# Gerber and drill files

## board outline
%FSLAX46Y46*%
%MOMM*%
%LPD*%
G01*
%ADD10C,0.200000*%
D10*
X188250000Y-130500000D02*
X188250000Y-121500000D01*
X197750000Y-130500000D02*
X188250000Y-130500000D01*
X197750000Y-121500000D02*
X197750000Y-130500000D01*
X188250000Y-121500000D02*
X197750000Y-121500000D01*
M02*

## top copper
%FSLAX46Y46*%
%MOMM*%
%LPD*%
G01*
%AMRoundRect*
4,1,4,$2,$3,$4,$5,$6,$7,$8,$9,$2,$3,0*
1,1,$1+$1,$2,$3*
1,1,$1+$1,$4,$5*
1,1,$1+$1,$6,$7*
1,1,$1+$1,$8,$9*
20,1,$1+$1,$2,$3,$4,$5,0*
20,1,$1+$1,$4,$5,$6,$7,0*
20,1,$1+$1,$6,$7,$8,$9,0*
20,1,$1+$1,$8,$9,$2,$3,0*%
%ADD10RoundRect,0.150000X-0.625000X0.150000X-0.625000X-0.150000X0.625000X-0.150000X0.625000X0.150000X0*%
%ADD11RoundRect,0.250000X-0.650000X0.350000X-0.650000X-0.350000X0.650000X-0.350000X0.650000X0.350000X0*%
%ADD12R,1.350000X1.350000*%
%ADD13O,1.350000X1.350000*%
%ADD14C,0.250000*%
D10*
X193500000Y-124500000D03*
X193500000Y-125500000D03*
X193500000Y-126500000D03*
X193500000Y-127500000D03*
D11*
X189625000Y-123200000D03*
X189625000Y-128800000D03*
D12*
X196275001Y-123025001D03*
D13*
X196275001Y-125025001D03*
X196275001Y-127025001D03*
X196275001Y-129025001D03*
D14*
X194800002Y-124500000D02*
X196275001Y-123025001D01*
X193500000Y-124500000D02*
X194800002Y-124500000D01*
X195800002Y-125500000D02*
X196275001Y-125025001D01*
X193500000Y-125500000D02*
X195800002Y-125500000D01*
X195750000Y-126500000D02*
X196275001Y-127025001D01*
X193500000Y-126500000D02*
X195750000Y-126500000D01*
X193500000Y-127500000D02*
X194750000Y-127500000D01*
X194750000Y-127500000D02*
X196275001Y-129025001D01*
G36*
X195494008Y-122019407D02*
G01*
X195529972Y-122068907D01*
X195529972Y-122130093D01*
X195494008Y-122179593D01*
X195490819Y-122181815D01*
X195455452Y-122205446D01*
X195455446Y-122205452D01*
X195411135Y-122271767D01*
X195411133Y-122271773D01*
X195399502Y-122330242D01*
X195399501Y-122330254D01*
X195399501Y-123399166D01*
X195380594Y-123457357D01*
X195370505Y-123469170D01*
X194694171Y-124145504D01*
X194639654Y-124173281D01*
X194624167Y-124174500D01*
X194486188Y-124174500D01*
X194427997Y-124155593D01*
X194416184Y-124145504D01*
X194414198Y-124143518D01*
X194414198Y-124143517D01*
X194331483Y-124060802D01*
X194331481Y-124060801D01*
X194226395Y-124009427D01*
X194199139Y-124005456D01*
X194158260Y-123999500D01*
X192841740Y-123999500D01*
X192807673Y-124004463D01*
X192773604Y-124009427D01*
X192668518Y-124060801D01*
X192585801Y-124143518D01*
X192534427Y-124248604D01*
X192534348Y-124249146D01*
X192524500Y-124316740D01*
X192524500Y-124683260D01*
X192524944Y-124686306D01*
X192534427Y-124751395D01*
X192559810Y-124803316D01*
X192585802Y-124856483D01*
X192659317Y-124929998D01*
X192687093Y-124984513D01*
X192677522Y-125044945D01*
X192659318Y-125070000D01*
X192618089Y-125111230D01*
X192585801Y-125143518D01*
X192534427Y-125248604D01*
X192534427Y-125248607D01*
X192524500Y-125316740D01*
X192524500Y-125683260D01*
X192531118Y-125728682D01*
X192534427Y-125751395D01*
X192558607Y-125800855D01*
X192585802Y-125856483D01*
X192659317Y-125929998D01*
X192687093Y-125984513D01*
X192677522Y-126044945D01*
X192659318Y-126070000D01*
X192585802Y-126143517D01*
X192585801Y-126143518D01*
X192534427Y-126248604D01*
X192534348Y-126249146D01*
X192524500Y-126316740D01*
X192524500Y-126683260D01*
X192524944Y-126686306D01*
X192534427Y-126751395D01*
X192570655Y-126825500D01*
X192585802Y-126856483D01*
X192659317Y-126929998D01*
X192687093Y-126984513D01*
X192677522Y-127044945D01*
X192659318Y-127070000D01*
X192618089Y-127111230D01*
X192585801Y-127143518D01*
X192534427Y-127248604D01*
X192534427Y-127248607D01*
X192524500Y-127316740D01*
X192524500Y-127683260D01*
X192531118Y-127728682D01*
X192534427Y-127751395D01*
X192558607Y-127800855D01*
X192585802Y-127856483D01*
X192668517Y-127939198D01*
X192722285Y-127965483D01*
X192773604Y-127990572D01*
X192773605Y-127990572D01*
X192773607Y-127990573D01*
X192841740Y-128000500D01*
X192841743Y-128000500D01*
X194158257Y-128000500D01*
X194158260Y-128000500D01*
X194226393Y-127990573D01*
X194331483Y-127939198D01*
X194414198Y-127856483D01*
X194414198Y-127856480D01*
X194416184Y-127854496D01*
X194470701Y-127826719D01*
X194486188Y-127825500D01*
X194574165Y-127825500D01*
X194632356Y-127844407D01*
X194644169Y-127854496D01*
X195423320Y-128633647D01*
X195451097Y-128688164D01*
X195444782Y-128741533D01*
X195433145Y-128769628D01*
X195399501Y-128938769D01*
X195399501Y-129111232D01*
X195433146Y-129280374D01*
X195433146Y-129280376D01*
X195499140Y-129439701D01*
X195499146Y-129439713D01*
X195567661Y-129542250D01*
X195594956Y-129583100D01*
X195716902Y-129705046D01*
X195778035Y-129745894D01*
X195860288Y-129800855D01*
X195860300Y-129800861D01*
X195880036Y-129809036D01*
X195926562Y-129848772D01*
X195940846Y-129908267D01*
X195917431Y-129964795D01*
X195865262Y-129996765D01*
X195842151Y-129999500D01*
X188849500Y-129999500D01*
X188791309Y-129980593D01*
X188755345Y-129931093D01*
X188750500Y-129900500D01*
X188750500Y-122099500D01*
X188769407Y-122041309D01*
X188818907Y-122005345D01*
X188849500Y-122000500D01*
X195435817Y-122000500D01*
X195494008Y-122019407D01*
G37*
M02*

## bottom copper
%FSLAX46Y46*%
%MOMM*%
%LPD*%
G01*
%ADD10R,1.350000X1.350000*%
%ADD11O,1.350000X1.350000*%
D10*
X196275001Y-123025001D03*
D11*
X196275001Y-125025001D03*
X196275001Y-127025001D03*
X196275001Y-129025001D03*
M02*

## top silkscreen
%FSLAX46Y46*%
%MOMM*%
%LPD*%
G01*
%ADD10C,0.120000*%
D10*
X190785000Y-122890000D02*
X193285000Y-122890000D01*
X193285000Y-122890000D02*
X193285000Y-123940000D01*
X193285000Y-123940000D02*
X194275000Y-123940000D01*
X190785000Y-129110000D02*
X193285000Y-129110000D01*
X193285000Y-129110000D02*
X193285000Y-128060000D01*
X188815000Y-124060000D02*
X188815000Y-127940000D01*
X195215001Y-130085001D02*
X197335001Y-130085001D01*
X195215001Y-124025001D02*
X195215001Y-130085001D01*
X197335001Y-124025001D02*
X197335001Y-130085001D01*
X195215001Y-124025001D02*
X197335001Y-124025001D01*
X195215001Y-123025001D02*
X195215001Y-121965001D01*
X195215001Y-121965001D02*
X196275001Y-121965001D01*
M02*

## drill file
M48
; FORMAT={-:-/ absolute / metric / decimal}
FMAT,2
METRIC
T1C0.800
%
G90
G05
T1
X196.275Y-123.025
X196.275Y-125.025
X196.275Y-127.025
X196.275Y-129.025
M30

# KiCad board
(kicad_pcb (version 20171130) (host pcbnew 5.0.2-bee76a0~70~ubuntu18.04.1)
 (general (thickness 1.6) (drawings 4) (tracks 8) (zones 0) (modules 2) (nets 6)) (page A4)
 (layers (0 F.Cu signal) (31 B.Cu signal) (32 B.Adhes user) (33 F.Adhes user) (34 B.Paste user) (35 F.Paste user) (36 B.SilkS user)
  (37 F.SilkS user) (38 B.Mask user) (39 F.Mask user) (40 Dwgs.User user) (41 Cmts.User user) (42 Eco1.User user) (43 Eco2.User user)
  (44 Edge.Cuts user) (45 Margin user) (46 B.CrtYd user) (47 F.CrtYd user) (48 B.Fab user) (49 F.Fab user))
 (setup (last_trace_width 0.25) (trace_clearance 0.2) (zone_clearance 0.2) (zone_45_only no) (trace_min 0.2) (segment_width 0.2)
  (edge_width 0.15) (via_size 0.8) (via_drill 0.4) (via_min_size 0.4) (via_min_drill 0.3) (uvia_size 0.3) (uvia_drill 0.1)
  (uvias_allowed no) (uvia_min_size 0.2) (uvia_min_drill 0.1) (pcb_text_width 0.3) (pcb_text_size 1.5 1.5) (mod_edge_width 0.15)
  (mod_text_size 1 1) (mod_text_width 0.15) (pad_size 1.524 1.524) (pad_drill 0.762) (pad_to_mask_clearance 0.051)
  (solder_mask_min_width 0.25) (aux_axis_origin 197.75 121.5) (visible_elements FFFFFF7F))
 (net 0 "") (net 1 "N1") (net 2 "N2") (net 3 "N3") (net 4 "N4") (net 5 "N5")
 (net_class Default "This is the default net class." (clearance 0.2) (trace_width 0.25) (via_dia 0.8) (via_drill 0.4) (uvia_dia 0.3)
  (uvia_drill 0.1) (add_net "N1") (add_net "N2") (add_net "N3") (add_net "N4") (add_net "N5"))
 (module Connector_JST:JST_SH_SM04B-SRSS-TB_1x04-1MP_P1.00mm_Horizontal (layer F.Cu) (at 191.5 126 270)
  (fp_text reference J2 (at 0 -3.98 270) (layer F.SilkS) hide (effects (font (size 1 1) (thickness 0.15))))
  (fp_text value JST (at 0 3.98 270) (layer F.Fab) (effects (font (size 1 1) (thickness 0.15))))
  (fp_line (start -3.11 0.715) (end -3.11 -1.785) (layer F.SilkS) (width 0.12))
  (fp_line (start -3.11 -1.785) (end -2.06 -1.785) (layer F.SilkS) (width 0.12))
  (fp_line (start -2.06 -1.785) (end -2.06 -2.775) (layer F.SilkS) (width 0.12))
  (fp_line (start 3.11 0.715) (end 3.11 -1.785) (layer F.SilkS) (width 0.12))
  (fp_line (start 3.11 -1.785) (end 2.06 -1.785) (layer F.SilkS) (width 0.12))
  (fp_line (start -1.94 2.685) (end 1.94 2.685) (layer F.SilkS) (width 0.12))
  (pad 1 smd roundrect (at -1.5 -2 270) (size 0.6 1.55) (layers F.Cu F.Paste F.Mask) (roundrect_rratio 0.25) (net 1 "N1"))
  (pad 2 smd roundrect (at -0.5 -2 270) (size 0.6 1.55) (layers F.Cu F.Paste F.Mask) (roundrect_rratio 0.25) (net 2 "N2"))
  (pad 3 smd roundrect (at 0.5 -2 270) (size 0.6 1.55) (layers F.Cu F.Paste F.Mask) (roundrect_rratio 0.25) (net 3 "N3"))
  (pad 4 smd roundrect (at 1.5 -2 270) (size 0.6 1.55) (layers F.Cu F.Paste F.Mask) (roundrect_rratio 0.25) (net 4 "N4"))
  (pad MP smd roundrect (at -2.8 1.875 270) (size 1.2 1.8) (layers F.Cu F.Paste F.Mask) (roundrect_rratio 0.208333) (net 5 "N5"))
  (pad MP smd roundrect (at 2.8 1.875 270) (size 1.2 1.8) (layers F.Cu F.Paste F.Mask) (roundrect_rratio 0.208333) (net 5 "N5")))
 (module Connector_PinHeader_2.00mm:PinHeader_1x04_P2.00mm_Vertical (layer F.Cu) (at 196.275001 123.025001)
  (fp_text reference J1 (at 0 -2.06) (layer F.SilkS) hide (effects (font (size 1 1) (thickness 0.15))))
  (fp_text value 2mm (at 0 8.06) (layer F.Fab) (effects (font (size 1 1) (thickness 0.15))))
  (fp_line (start -1.06 7.06) (end 1.06 7.06) (layer F.SilkS) (width 0.12))
  (fp_line (start -1.06 1) (end -1.06 7.06) (layer F.SilkS) (width 0.12))
  (fp_line (start 1.06 1) (end 1.06 7.06) (layer F.SilkS) (width 0.12))
  (fp_line (start -1.06 1) (end 1.06 1) (layer F.SilkS) (width 0.12))
  (fp_line (start -1.06 0) (end -1.06 -1.06) (layer F.SilkS) (width 0.12))
  (fp_line (start -1.06 -1.06) (end 0 -1.06) (layer F.SilkS) (width 0.12))
  (pad 1 thru_hole rect (at 0 0) (size 1.35 1.35) (drill 0.8) (layers *.Cu *.Mask) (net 1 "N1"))
  (pad 2 thru_hole oval (at 0 2) (size 1.35 1.35) (drill 0.8) (layers *.Cu *.Mask) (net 2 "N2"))
  (pad 3 thru_hole oval (at 0 4) (size 1.35 1.35) (drill 0.8) (layers *.Cu *.Mask) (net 3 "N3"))
  (pad 4 thru_hole oval (at 0 6) (size 1.35 1.35) (drill 0.8) (layers *.Cu *.Mask) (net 4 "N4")))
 (gr_line (start 188.25 130.5) (end 188.25 121.5) (layer Edge.Cuts) (width 0.2))
 (gr_line (start 197.75 130.5) (end 188.25 130.5) (layer Edge.Cuts) (width 0.2))
 (gr_line (start 197.75 121.5) (end 197.75 130.5) (layer Edge.Cuts) (width 0.2))
 (gr_line (start 188.25 121.5) (end 197.75 121.5) (layer Edge.Cuts) (width 0.2))
 (segment (start 194.800002 124.5) (end 196.275001 123.025001) (width 0.25) (layer F.Cu) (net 1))
 (segment (start 193.5 124.5) (end 194.800002 124.5) (width 0.25) (layer F.Cu) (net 1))
 (segment (start 195.800002 125.5) (end 196.275001 125.025001) (width 0.25) (layer F.Cu) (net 2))
 (segment (start 193.5 125.5) (end 195.800002 125.5) (width 0.25) (layer F.Cu) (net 2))
 (segment (start 195.75 126.5) (end 196.275001 127.025001) (width 0.25) (layer F.Cu) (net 3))
 (segment (start 193.5 126.5) (end 195.75 126.5) (width 0.25) (layer F.Cu) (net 3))
 (segment (start 193.5 127.5) (end 194.75 127.5) (width 0.25) (layer F.Cu) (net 4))
 (segment (start 194.75 127.5) (end 196.275001 129.025001) (width 0.25) (layer F.Cu) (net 4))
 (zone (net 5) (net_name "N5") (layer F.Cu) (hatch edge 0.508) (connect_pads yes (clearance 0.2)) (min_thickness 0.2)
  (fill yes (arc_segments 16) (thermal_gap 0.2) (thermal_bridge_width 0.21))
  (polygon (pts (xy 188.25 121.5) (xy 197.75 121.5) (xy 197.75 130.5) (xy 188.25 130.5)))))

